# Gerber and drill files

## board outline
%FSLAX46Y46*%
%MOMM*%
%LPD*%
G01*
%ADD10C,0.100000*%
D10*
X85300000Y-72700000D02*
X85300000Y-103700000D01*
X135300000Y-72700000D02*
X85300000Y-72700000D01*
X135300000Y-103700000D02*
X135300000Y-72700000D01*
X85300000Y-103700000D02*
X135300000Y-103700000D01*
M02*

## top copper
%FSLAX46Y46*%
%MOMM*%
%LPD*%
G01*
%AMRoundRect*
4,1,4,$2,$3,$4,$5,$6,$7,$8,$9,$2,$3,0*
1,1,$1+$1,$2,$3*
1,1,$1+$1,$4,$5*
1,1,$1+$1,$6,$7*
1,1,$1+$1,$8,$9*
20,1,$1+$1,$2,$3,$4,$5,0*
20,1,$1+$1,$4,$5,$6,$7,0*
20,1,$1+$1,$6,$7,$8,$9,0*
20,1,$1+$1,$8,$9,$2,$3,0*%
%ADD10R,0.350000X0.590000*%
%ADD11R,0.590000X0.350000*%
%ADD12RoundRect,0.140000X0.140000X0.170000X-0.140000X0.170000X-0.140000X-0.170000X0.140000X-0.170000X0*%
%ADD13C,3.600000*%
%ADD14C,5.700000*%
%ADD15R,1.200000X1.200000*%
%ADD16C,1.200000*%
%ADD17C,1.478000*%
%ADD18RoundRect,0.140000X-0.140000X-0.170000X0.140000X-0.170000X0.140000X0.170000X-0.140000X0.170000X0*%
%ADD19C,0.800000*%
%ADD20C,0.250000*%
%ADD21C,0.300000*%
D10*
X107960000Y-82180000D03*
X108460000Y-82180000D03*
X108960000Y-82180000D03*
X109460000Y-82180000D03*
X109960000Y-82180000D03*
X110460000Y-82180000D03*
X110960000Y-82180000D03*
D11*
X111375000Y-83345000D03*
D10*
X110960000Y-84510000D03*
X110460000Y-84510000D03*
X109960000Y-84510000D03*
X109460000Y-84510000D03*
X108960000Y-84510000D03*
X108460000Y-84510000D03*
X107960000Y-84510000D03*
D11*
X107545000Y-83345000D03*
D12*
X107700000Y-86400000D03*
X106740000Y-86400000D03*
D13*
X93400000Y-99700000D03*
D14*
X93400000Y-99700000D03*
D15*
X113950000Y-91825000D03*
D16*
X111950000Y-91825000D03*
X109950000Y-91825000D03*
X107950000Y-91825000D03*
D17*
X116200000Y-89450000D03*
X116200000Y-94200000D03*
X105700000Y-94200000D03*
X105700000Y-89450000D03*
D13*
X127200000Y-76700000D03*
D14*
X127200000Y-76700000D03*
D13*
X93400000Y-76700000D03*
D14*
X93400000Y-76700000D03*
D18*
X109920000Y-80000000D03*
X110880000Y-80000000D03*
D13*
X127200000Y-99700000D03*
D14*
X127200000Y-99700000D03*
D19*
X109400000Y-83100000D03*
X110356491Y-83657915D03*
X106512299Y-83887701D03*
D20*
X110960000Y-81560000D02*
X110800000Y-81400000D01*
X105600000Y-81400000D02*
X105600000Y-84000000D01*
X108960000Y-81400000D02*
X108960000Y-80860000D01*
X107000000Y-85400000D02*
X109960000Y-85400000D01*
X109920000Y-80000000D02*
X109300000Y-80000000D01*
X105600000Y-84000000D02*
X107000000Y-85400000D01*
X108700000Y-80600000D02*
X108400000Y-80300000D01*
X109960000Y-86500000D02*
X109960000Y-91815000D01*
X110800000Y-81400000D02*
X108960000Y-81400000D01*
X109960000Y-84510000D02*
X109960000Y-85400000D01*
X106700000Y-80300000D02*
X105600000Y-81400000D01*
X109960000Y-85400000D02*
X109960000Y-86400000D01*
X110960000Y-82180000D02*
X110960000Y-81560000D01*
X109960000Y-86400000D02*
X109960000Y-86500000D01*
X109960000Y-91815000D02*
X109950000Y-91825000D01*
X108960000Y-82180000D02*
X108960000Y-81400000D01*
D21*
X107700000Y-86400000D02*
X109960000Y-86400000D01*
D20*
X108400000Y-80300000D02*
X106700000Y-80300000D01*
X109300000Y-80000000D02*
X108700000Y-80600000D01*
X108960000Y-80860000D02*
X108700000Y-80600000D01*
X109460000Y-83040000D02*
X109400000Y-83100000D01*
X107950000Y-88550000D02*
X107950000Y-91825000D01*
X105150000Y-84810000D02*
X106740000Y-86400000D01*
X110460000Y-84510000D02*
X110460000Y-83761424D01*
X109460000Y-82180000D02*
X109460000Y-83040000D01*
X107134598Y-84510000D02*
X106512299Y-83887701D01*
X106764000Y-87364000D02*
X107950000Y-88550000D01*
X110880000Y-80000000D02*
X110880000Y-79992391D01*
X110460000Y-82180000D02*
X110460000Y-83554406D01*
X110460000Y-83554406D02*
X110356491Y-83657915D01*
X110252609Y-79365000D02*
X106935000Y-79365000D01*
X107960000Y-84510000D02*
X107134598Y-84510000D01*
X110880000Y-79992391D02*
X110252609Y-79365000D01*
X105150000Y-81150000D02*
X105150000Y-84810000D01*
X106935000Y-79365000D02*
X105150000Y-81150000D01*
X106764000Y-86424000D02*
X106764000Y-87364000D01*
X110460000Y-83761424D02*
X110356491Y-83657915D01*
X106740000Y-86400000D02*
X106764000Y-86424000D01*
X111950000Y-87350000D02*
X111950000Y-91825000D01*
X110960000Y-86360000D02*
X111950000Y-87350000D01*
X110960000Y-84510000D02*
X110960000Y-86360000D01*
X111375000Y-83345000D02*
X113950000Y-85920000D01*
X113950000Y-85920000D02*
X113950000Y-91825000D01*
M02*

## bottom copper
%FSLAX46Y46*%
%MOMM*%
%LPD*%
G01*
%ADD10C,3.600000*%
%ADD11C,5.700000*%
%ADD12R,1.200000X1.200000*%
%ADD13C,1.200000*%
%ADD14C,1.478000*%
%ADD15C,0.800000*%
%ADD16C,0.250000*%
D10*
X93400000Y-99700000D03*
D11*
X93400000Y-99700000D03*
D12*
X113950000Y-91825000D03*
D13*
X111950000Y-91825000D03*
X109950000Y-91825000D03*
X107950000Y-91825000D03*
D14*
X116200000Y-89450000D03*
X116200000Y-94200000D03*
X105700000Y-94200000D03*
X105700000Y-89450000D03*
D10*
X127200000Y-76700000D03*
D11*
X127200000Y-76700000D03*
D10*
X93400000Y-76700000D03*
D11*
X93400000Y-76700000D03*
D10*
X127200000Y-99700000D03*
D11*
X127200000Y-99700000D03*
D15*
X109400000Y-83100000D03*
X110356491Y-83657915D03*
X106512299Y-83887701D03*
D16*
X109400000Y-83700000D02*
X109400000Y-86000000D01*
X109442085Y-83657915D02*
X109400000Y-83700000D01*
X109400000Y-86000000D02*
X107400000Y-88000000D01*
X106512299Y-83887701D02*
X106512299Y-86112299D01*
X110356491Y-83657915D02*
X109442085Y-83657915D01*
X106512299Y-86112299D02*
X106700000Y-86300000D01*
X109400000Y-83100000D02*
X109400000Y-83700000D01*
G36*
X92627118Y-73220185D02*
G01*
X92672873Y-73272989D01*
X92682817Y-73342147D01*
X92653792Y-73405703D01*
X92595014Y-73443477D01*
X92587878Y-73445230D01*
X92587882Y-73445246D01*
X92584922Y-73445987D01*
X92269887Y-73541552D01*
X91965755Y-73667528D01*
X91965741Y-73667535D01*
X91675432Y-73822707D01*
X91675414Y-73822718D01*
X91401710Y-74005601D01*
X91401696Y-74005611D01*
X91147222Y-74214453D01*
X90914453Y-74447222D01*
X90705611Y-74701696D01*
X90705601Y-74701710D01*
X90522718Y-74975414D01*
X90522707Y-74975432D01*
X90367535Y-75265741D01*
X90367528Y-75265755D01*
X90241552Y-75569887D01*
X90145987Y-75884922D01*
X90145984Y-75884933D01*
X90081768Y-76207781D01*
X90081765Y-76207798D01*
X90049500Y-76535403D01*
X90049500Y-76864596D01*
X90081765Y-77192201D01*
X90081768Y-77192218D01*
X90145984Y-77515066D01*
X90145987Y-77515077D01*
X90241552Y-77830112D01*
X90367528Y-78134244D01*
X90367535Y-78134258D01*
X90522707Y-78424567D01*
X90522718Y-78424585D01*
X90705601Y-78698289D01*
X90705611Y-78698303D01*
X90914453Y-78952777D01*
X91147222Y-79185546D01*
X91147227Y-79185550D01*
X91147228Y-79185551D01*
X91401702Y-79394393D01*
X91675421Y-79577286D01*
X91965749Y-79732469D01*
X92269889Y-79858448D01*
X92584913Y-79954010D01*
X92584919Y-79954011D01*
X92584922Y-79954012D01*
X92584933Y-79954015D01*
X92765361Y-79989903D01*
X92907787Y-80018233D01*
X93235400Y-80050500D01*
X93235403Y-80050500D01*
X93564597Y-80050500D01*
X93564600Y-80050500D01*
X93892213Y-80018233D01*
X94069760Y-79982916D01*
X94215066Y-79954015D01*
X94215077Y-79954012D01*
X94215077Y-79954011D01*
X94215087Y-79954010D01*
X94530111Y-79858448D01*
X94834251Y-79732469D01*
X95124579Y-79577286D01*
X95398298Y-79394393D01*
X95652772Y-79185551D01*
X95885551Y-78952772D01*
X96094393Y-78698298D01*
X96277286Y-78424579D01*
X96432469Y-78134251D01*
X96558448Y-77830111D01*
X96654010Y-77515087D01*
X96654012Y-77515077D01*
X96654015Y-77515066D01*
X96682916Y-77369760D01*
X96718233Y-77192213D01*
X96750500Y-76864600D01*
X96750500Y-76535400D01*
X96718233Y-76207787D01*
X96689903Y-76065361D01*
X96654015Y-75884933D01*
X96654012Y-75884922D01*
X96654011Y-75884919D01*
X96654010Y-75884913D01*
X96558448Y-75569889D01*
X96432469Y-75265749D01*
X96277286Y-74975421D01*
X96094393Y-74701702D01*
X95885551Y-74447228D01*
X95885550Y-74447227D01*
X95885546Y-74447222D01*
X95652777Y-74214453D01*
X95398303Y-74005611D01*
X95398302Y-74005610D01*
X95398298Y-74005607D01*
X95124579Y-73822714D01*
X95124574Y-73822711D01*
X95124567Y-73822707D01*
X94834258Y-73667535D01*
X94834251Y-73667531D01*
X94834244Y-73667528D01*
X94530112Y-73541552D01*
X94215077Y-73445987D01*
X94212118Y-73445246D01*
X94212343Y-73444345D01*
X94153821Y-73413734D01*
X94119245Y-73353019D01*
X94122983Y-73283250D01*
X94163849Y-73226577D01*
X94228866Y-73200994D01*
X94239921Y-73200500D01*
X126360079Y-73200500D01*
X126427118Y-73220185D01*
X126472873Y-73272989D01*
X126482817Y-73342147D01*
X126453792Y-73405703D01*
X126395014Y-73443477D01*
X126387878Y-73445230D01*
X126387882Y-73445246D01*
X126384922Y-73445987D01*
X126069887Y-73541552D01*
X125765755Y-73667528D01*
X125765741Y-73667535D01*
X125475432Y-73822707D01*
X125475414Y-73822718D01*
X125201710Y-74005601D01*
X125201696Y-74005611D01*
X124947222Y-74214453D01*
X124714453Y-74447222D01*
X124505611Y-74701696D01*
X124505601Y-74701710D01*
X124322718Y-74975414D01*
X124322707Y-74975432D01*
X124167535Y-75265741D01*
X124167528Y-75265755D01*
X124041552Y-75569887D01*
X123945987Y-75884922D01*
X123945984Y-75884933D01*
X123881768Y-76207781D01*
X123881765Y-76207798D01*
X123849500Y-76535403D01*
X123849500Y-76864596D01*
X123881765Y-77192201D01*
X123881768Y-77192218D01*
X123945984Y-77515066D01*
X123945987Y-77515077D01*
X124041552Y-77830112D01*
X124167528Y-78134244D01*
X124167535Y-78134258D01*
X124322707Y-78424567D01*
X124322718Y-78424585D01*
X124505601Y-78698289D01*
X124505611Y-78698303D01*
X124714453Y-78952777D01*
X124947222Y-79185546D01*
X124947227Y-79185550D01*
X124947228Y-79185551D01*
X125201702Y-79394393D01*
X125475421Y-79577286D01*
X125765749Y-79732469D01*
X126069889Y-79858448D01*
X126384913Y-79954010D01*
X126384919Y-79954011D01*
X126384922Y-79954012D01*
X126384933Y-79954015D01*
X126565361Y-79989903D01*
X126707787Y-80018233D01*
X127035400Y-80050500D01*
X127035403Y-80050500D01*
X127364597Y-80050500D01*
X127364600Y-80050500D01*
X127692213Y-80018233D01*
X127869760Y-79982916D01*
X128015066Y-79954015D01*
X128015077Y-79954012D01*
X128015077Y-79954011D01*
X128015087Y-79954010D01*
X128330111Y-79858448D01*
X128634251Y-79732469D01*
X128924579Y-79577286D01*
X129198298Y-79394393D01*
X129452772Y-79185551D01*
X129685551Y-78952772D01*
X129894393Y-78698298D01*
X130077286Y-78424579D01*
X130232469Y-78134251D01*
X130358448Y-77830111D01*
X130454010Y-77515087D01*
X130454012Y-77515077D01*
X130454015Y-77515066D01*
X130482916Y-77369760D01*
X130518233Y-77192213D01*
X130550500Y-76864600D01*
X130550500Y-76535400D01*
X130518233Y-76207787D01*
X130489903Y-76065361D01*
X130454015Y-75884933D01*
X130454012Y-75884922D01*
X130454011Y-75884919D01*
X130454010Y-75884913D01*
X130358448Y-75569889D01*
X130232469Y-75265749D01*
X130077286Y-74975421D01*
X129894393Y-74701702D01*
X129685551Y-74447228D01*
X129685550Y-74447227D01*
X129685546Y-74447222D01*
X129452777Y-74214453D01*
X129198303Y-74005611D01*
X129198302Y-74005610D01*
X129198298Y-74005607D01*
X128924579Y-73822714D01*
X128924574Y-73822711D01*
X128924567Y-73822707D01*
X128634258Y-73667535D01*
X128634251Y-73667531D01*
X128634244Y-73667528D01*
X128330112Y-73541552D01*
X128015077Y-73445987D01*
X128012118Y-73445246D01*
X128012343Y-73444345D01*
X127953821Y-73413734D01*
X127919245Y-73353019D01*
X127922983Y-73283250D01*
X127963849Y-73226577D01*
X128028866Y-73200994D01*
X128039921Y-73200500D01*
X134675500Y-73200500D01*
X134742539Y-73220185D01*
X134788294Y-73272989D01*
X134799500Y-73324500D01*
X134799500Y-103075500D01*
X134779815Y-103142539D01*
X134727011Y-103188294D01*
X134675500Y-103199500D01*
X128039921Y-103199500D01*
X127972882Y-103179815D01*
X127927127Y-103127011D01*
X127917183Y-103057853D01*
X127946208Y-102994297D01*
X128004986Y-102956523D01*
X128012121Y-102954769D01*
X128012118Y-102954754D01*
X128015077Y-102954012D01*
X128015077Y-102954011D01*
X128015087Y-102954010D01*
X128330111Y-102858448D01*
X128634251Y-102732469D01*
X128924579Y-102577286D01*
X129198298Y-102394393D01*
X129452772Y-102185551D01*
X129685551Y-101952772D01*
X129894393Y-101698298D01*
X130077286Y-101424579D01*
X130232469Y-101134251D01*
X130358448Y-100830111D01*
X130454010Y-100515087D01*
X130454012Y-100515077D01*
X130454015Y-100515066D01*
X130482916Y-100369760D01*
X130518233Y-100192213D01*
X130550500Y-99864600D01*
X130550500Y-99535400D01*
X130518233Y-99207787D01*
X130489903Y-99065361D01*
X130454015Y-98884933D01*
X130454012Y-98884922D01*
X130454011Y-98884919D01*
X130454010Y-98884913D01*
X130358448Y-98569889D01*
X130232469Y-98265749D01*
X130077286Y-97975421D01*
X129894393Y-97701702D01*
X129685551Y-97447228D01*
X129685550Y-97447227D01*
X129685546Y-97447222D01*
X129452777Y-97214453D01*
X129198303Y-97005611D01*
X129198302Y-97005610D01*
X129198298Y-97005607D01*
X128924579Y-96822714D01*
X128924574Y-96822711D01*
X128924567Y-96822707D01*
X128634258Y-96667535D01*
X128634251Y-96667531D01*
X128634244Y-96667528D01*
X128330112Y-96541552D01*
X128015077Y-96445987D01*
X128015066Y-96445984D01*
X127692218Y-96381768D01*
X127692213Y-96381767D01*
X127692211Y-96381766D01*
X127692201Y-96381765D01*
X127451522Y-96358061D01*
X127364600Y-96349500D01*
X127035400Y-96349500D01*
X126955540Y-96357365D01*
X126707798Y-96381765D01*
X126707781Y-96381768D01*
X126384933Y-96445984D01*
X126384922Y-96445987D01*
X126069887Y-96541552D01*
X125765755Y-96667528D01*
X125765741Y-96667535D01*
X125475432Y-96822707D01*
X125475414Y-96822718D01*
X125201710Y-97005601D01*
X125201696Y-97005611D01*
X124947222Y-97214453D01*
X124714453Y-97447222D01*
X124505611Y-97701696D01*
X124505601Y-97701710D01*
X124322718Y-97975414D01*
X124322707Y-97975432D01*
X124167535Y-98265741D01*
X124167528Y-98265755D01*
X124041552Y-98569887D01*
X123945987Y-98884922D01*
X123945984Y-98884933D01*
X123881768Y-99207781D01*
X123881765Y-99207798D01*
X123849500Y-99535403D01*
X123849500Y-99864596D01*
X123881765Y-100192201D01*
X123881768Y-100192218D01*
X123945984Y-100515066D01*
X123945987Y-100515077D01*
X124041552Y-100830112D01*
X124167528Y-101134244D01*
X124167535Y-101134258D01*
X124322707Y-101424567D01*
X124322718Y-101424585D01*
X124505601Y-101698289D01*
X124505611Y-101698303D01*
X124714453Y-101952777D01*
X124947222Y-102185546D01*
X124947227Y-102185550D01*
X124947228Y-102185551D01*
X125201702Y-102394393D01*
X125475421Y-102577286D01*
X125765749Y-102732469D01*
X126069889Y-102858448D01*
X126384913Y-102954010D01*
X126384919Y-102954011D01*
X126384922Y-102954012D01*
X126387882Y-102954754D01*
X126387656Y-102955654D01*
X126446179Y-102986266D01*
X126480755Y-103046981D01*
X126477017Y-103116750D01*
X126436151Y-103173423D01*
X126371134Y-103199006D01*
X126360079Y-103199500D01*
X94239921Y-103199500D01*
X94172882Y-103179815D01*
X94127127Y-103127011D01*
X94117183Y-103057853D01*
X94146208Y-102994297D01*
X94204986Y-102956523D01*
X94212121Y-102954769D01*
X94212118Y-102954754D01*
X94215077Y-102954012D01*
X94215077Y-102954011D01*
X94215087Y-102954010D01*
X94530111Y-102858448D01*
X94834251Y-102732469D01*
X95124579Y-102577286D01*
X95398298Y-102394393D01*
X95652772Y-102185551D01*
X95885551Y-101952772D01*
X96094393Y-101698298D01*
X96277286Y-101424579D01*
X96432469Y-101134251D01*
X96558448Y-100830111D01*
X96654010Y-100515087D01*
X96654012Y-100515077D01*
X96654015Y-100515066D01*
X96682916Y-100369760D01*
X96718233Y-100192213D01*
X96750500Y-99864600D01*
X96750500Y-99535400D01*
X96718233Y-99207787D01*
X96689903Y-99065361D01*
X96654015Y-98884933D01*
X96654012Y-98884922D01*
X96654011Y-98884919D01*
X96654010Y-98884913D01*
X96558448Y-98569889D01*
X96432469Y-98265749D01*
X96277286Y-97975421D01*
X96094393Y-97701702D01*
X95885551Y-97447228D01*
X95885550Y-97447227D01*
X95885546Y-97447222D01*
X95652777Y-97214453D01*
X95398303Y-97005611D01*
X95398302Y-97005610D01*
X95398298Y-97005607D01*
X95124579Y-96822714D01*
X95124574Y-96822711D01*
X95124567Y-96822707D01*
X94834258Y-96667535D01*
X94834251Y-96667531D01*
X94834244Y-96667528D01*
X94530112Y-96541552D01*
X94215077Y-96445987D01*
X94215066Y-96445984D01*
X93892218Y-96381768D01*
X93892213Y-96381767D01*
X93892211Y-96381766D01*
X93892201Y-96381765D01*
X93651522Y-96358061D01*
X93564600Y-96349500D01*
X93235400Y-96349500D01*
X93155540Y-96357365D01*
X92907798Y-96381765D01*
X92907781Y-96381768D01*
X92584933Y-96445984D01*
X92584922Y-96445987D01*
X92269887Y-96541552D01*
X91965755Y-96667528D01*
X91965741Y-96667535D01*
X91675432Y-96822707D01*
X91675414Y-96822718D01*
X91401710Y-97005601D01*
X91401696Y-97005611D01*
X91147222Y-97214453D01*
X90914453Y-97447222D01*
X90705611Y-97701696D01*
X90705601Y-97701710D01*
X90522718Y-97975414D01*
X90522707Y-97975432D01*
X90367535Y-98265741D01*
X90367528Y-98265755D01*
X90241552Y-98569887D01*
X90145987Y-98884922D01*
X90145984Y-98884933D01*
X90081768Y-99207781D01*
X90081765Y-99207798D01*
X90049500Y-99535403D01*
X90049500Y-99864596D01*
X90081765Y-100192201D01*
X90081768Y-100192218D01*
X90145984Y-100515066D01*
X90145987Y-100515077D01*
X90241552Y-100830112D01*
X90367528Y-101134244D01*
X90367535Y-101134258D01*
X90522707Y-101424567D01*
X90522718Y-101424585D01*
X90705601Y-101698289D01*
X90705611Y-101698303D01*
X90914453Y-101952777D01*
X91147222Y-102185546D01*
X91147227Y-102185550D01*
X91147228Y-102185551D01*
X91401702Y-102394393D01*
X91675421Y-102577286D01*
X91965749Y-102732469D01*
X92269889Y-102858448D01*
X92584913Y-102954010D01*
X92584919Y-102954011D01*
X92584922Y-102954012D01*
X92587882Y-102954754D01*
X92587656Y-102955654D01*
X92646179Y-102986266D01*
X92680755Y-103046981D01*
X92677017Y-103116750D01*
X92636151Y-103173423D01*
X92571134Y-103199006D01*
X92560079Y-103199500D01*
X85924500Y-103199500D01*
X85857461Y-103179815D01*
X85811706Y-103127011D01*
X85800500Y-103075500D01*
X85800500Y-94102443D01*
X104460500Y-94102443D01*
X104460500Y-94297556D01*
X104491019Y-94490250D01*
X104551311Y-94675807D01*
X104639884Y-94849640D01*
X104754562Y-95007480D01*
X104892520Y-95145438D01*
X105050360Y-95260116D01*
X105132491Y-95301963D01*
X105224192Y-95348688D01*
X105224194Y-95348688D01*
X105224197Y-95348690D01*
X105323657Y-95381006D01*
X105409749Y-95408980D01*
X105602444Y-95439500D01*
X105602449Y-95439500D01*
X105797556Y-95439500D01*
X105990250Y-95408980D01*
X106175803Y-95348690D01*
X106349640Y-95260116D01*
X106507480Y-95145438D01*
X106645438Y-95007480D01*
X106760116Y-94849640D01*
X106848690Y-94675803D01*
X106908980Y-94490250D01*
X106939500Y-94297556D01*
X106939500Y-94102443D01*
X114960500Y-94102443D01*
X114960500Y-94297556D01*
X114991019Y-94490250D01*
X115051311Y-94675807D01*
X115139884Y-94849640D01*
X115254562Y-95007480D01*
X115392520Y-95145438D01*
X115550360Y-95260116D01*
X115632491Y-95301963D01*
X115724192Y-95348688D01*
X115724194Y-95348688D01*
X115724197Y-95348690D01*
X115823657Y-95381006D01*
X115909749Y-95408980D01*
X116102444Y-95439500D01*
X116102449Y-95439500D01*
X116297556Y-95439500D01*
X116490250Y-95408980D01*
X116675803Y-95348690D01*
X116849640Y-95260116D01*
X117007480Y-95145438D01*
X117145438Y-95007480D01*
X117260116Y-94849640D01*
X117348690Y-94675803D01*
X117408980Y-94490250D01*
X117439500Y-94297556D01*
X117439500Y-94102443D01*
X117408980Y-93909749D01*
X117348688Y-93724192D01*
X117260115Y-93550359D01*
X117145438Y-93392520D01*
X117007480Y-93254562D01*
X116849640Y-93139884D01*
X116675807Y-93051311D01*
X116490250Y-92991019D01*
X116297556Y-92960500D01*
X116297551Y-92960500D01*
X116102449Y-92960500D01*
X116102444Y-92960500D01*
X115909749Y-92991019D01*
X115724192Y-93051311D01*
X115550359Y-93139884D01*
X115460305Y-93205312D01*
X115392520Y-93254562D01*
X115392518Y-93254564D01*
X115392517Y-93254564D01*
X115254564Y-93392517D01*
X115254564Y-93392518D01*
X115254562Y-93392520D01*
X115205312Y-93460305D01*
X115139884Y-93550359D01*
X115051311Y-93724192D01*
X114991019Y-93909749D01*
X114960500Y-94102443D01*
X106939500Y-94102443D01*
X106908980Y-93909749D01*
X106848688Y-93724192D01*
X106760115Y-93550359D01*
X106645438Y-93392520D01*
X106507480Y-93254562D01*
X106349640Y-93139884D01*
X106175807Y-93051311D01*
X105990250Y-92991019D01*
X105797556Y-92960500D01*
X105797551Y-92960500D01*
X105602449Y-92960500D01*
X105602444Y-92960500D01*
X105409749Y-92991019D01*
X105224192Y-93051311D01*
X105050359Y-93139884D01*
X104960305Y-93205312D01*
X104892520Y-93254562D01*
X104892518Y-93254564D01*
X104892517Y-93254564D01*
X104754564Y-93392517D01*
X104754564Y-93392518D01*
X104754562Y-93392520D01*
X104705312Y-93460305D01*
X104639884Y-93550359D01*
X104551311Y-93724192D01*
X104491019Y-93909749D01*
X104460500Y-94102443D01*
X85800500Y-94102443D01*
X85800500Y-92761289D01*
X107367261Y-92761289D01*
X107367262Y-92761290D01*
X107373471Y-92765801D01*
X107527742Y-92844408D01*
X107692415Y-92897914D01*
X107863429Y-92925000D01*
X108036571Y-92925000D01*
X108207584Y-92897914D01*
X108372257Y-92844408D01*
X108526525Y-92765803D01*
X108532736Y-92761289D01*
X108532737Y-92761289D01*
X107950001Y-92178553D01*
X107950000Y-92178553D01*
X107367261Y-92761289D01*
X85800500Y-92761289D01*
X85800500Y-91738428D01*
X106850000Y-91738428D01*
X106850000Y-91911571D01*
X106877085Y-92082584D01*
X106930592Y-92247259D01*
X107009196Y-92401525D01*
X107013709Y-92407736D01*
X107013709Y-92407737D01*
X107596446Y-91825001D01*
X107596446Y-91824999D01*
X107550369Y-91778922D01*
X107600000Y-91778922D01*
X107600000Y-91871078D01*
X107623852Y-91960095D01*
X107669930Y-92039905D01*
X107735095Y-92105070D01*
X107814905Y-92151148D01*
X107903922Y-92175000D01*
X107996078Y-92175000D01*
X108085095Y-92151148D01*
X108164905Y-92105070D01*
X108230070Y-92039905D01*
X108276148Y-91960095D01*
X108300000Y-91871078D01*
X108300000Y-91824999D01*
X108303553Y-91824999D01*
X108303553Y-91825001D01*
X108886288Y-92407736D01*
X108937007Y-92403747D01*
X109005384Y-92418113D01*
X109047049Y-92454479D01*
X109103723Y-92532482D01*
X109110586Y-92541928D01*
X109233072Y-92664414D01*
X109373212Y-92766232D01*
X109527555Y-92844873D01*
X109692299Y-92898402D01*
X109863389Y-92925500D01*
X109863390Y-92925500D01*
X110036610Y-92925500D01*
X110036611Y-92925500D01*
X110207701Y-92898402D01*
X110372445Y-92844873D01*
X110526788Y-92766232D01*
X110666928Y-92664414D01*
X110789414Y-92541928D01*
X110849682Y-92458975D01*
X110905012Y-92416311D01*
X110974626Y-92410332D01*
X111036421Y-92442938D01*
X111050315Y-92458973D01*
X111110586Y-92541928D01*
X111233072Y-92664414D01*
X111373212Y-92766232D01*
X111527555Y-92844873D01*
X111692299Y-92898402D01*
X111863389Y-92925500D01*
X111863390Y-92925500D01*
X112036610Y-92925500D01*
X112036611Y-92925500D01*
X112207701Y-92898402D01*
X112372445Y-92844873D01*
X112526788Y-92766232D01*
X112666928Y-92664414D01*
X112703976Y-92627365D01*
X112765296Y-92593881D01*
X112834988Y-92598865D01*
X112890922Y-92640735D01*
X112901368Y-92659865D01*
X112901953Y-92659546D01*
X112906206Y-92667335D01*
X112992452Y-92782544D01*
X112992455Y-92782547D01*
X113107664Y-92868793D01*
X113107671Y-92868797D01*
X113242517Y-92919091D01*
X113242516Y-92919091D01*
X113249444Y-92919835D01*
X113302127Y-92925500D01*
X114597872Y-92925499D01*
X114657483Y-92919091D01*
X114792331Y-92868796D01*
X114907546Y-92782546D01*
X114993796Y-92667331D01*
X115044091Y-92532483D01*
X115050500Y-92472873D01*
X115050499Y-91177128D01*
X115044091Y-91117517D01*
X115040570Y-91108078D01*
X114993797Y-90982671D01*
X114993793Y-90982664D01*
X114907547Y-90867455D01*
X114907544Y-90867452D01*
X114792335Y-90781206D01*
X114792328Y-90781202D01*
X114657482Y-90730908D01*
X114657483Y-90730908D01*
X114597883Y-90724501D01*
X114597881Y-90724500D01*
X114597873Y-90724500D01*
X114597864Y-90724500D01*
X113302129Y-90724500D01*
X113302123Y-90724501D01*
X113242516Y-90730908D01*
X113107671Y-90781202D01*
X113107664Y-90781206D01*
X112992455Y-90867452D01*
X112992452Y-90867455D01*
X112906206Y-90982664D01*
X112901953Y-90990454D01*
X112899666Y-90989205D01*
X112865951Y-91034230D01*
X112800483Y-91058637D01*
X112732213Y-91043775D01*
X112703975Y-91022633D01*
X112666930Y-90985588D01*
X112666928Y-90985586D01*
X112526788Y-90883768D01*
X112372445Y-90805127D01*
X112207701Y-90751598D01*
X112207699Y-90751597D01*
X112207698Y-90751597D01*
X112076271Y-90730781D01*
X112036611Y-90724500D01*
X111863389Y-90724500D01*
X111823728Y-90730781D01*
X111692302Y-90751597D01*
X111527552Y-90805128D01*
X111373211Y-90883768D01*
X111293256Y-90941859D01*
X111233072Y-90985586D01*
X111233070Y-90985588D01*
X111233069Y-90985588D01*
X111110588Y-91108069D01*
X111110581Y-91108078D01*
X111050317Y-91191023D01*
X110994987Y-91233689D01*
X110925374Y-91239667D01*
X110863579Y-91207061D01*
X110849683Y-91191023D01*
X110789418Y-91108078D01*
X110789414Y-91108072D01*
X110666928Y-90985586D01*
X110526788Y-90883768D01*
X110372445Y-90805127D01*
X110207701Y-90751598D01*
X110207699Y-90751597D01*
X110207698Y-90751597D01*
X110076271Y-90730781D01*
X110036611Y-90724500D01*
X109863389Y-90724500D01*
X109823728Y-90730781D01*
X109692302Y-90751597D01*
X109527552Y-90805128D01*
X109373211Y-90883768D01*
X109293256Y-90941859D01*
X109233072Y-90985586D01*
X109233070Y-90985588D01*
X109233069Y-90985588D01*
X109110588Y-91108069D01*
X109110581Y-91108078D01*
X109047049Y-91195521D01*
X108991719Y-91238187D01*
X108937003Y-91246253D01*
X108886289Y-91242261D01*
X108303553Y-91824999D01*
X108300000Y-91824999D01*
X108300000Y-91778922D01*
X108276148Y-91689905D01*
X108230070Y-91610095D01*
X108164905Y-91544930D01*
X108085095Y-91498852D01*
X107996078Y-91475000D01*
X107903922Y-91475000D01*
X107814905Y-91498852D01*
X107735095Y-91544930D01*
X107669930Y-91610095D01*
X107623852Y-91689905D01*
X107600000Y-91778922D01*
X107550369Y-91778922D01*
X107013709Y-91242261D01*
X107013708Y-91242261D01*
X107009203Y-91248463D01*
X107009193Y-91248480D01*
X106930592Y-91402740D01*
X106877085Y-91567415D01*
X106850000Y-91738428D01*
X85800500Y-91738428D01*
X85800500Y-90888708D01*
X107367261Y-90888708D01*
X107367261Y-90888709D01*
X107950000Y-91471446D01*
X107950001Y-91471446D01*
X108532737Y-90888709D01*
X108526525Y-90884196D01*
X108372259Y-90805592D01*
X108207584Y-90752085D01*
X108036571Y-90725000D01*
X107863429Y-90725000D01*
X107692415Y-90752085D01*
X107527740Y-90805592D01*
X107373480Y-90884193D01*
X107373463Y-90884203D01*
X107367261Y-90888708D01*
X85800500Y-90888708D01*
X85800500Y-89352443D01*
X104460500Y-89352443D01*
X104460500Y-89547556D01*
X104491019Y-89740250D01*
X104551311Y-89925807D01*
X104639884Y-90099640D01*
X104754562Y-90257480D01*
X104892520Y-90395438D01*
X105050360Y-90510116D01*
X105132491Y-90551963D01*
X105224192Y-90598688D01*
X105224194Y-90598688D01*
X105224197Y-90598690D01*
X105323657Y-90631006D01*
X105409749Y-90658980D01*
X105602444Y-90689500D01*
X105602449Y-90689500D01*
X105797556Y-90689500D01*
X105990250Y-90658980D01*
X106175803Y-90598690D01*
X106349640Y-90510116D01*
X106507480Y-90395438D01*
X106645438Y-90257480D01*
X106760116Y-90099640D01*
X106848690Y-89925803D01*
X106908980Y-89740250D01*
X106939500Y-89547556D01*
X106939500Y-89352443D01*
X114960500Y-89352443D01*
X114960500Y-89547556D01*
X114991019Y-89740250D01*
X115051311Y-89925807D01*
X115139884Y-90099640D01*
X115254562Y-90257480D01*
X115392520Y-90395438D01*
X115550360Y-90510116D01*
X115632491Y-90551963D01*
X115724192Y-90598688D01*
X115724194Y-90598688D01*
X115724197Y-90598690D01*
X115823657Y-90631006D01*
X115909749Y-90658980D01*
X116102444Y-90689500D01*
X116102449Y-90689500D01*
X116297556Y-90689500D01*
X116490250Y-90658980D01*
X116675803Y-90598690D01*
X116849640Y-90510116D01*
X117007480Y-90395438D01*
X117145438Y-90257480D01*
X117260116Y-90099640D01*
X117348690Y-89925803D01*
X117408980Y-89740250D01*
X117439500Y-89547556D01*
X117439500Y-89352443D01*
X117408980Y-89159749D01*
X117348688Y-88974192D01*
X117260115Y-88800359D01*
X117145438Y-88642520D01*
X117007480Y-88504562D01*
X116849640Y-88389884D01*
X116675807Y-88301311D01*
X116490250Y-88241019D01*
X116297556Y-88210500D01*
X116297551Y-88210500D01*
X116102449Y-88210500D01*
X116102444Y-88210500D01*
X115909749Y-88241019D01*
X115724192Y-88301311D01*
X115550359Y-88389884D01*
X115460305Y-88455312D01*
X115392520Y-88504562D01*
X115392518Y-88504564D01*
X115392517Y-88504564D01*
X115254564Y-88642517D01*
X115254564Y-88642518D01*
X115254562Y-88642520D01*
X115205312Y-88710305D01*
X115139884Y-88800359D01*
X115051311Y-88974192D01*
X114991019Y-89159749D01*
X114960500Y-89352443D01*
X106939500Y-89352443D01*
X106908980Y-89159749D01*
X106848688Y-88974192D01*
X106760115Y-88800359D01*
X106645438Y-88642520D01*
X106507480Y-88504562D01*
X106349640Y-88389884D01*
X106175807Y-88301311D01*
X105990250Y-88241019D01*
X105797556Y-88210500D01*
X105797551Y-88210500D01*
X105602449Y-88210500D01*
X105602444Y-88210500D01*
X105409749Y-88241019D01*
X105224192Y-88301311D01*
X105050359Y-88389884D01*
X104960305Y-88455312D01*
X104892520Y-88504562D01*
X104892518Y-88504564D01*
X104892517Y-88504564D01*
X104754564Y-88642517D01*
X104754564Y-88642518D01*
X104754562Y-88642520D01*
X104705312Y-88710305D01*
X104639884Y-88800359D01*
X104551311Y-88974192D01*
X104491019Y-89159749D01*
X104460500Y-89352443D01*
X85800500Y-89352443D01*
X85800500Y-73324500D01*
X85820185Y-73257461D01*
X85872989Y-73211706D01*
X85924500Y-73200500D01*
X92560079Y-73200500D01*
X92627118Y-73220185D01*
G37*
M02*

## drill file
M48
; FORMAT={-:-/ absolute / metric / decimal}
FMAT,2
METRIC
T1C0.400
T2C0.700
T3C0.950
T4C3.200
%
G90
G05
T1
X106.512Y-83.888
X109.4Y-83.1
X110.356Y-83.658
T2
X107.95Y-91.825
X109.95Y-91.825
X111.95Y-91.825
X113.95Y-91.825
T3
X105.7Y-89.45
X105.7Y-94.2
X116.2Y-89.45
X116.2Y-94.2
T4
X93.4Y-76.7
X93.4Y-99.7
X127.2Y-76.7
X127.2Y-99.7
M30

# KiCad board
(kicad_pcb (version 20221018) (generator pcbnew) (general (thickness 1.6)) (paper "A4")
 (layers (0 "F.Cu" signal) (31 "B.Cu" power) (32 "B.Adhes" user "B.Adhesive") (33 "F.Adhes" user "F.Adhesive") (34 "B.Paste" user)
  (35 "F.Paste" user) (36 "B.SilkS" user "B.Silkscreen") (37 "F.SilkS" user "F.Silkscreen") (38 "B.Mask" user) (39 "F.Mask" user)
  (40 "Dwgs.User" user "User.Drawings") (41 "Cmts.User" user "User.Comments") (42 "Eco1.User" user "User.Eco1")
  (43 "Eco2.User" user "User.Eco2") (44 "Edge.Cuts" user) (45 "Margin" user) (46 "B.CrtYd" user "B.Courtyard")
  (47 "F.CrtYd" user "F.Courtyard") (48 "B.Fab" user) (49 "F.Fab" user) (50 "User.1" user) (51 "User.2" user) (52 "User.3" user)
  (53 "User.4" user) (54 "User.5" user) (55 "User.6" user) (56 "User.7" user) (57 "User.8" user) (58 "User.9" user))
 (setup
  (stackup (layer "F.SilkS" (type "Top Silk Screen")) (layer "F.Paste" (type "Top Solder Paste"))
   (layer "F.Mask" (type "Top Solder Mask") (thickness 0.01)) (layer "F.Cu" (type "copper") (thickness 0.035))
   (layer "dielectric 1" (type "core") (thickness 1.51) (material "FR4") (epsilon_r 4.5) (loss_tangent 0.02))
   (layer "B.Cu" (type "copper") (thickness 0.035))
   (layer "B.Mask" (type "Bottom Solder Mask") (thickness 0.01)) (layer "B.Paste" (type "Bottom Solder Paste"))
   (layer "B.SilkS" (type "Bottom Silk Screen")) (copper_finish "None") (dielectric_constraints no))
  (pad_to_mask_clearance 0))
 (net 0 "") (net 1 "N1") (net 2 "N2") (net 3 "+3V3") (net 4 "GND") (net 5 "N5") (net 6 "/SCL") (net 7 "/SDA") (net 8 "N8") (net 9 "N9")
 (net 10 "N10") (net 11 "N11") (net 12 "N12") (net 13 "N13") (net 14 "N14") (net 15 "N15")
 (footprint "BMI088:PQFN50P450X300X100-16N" (layer "F.Cu") (at 109.46 83.345)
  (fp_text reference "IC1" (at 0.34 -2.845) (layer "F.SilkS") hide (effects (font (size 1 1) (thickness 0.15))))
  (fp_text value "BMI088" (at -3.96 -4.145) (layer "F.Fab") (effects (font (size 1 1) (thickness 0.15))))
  (pad "1" smd rect (at -1.5 -1.165 270) (size 0.59 0.35) (layers "F.Cu" "F.Paste" "F.Mask") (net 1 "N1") (solder_mask_margin 0.102))
  (pad "2" smd rect (at -1 -1.165 270) (size 0.59 0.35) (layers "F.Cu" "F.Paste" "F.Mask") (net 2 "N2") (solder_mask_margin 0.102))
  (pad "3" smd rect (at -0.5 -1.165 270) (size 0.59 0.35) (layers "F.Cu" "F.Paste" "F.Mask") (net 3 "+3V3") (solder_mask_margin 0.102))
  (pad "4" smd rect (at 0 -1.165 270) (size 0.59 0.35) (layers "F.Cu" "F.Paste" "F.Mask") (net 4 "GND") (solder_mask_margin 0.102))
  (pad "5" smd rect (at 0.5 -1.165 270) (size 0.59 0.35) (layers "F.Cu" "F.Paste" "F.Mask") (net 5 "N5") (solder_mask_margin 0.102))
  (pad "6" smd rect (at 1 -1.165 270) (size 0.59 0.35) (layers "F.Cu" "F.Paste" "F.Mask") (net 4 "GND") (solder_mask_margin 0.102))
  (pad "7" smd rect (at 1.5 -1.165 270) (size 0.59 0.35) (layers "F.Cu" "F.Paste" "F.Mask") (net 3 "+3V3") (solder_mask_margin 0.102))
  (pad "8" smd rect (at 1.915 0 180) (size 0.59 0.35) (layers "F.Cu" "F.Paste" "F.Mask") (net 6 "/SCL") (solder_mask_margin 0.102))
  (pad "9" smd rect (at 1.5 1.165 90) (size 0.59 0.35) (layers "F.Cu" "F.Paste" "F.Mask") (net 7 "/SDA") (solder_mask_margin 0.102))
  (pad "10" smd rect (at 1 1.165 90) (size 0.59 0.35) (layers "F.Cu" "F.Paste" "F.Mask") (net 4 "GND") (solder_mask_margin 0.102))
  (pad "11" smd rect (at 0.5 1.165 90) (size 0.59 0.35) (layers "F.Cu" "F.Paste" "F.Mask") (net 3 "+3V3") (solder_mask_margin 0.102))
  (pad "12" smd rect (at 0 1.165 90) (size 0.59 0.35) (layers "F.Cu" "F.Paste" "F.Mask") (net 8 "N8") (solder_mask_margin 0.102))
  (pad "13" smd rect (at -0.5 1.165 90) (size 0.59 0.35) (layers "F.Cu" "F.Paste" "F.Mask") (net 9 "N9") (solder_mask_margin 0.102))
  (pad "14" smd rect (at -1 1.165 90) (size 0.59 0.35) (layers "F.Cu" "F.Paste" "F.Mask") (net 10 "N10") (solder_mask_margin 0.102))
  (pad "15" smd rect (at -1.5 1.165 90) (size 0.59 0.35) (layers "F.Cu" "F.Paste" "F.Mask") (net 4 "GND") (solder_mask_margin 0.102))
  (pad "16" smd rect (at -1.915 0) (size 0.59 0.35) (layers "F.Cu" "F.Paste" "F.Mask") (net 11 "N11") (solder_mask_margin 0.102)))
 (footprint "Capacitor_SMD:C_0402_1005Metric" (layer "F.Cu") (at 107.22 86.4 180)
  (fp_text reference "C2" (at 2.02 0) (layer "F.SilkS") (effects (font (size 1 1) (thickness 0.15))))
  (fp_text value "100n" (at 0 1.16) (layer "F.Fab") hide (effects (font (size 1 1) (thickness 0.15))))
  (pad "1" smd roundrect (at -0.48 0 180) (size 0.56 0.62) (layers "F.Cu" "F.Paste" "F.Mask") (roundrect_rratio 0.25) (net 3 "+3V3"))
  (pad "2" smd roundrect (at 0.48 0 180) (size 0.56 0.62) (layers "F.Cu" "F.Paste" "F.Mask") (roundrect_rratio 0.25) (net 4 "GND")))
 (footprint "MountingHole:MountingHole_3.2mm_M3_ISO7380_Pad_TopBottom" (layer "F.Cu") (at 93.4 99.7)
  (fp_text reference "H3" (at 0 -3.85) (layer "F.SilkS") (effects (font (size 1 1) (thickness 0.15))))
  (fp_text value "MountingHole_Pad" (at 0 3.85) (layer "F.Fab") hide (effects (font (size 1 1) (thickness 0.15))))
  (pad "1" thru_hole circle (at 0 0) (size 3.6 3.6) (drill 3.2) (layers "*.Cu" "*.Mask"))
  (pad "1" connect circle (at 0 0) (size 5.7 5.7) (layers "F.Cu" "F.Mask"))
  (pad "1" connect circle (at 0 0) (size 5.7 5.7) (layers "B.Cu" "B.Mask")))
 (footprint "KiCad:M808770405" (layer "F.Cu") (at 113.95 91.825)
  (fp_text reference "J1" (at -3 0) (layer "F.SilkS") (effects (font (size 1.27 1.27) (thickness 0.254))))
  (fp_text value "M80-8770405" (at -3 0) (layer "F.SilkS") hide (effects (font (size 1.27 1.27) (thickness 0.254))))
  (pad "1" thru_hole rect (at 0 0) (size 1.2 1.2) (drill 0.7) (layers "*.Cu" "*.Mask") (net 6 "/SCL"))
  (pad "2" thru_hole circle (at -2 0) (size 1.2 1.2) (drill 0.7) (layers "*.Cu" "*.Mask") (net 7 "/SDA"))
  (pad "3" thru_hole circle (at -4 0) (size 1.2 1.2) (drill 0.7) (layers "*.Cu" "*.Mask") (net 3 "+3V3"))
  (pad "4" thru_hole circle (at -6 0) (size 1.2 1.2) (drill 0.7) (layers "*.Cu" "*.Mask") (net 4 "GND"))
  (pad "MH1" thru_hole circle (at 2.25 -2.375) (size 1.478 1.478) (drill 0.95) (layers "*.Cu" "*.Mask") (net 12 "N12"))
  (pad "MH2" thru_hole circle (at 2.25 2.375) (size 1.478 1.478) (drill 0.95) (layers "*.Cu" "*.Mask") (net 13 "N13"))
  (pad "MH3" thru_hole circle (at -8.25 2.375) (size 1.478 1.478) (drill 0.95) (layers "*.Cu" "*.Mask") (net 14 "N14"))
  (pad "MH4" thru_hole circle (at -8.25 -2.375) (size 1.478 1.478) (drill 0.95) (layers "*.Cu" "*.Mask") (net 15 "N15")))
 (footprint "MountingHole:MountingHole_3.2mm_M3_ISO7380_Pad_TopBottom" (layer "F.Cu") (at 127.2 76.7)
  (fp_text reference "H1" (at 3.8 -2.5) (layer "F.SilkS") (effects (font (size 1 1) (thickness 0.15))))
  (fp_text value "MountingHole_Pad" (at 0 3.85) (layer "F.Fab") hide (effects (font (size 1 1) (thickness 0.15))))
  (pad "1" thru_hole circle (at 0 0) (size 3.6 3.6) (drill 3.2) (layers "*.Cu" "*.Mask"))
  (pad "1" connect circle (at 0 0) (size 5.7 5.7) (layers "F.Cu" "F.Mask"))
  (pad "1" connect circle (at 0 0) (size 5.7 5.7) (layers "B.Cu" "B.Mask")))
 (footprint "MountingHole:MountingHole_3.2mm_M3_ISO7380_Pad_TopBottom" (layer "F.Cu") (at 93.4 76.7)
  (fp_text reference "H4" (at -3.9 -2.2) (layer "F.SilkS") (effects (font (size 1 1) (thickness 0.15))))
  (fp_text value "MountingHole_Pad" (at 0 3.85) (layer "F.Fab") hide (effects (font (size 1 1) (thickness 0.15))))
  (pad "1" thru_hole circle (at 0 0) (size 3.6 3.6) (drill 3.2) (layers "*.Cu" "*.Mask"))
  (pad "1" connect circle (at 0 0) (size 5.7 5.7) (layers "F.Cu" "F.Mask"))
  (pad "1" connect circle (at 0 0) (size 5.7 5.7) (layers "B.Cu" "B.Mask")))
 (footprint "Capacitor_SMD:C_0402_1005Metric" (layer "F.Cu") (at 110.4 80)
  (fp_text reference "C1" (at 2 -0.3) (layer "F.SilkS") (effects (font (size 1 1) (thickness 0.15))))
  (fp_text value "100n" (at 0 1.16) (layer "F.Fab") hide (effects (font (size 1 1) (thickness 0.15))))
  (pad "1" smd roundrect (at -0.48 0) (size 0.56 0.62) (layers "F.Cu" "F.Paste" "F.Mask") (roundrect_rratio 0.25) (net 3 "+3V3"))
  (pad "2" smd roundrect (at 0.48 0) (size 0.56 0.62) (layers "F.Cu" "F.Paste" "F.Mask") (roundrect_rratio 0.25) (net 4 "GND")))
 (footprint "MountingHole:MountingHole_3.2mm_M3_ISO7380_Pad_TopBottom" (layer "F.Cu") (at 127.2 99.7)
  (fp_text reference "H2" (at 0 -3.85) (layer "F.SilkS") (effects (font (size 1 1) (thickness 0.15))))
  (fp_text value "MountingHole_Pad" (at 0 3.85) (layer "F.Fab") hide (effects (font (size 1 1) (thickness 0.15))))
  (pad "1" thru_hole circle (at 0 0) (size 3.6 3.6) (drill 3.2) (layers "*.Cu" "*.Mask"))
  (pad "1" connect circle (at 0 0) (size 5.7 5.7) (layers "F.Cu" "F.Mask"))
  (pad "1" connect circle (at 0 0) (size 5.7 5.7) (layers "B.Cu" "B.Mask")))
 (gr_line (start 85.3 72.7) (end 85.3 103.7) (stroke (width 0.1) (type default)) (layer "Edge.Cuts"))
 (gr_line (start 135.3 72.7) (end 85.3 72.7) (stroke (width 0.1) (type default)) (layer "Edge.Cuts"))
 (gr_line (start 135.3 103.7) (end 135.3 72.7) (stroke (width 0.1) (type default)) (layer "Edge.Cuts"))
 (gr_line (start 85.3 103.7) (end 135.3 103.7) (stroke (width 0.1) (type default)) (layer "Edge.Cuts"))
 (segment (start 110.96 81.56) (end 110.8 81.4) (width 0.25) (layer "F.Cu") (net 3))
 (segment (start 105.6 81.4) (end 105.6 84) (width 0.25) (layer "F.Cu") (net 3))
 (segment (start 108.96 81.4) (end 108.96 80.86) (width 0.25) (layer "F.Cu") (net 3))
 (segment (start 107 85.4) (end 109.96 85.4) (width 0.25) (layer "F.Cu") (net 3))
 (segment (start 109.92 80) (end 109.3 80) (width 0.25) (layer "F.Cu") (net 3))
 (segment (start 105.6 84) (end 107 85.4) (width 0.25) (layer "F.Cu") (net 3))
 (segment (start 108.7 80.6) (end 108.4 80.3) (width 0.25) (layer "F.Cu") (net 3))
 (segment (start 109.96 86.5) (end 109.96 91.815) (width 0.25) (layer "F.Cu") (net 3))
 (segment (start 110.8 81.4) (end 108.96 81.4) (width 0.25) (layer "F.Cu") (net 3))
 (segment (start 109.96 84.51) (end 109.96 85.4) (width 0.25) (layer "F.Cu") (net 3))
 (segment (start 106.7 80.3) (end 105.6 81.4) (width 0.25) (layer "F.Cu") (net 3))
 (segment (start 109.96 85.4) (end 109.96 86.4) (width 0.25) (layer "F.Cu") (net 3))
 (segment (start 110.96 82.18) (end 110.96 81.56) (width 0.25) (layer "F.Cu") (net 3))
 (segment (start 109.96 86.4) (end 109.96 86.5) (width 0.25) (layer "F.Cu") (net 3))
 (segment (start 109.96 91.815) (end 109.95 91.825) (width 0.25) (layer "F.Cu") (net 3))
 (segment (start 108.96 82.18) (end 108.96 81.4) (width 0.25) (layer "F.Cu") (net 3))
 (segment (start 107.7 86.4) (end 109.96 86.4) (width 0.3) (layer "F.Cu") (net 3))
 (segment (start 108.4 80.3) (end 106.7 80.3) (width 0.25) (layer "F.Cu") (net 3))
 (segment (start 109.3 80) (end 108.7 80.6) (width 0.25) (layer "F.Cu") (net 3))
 (segment (start 108.96 80.86) (end 108.7 80.6) (width 0.25) (layer "F.Cu") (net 3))
 (segment (start 109.46 83.04) (end 109.4 83.1) (width 0.25) (layer "F.Cu") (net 4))
 (segment (start 107.95 88.55) (end 107.95 91.825) (width 0.25) (layer "F.Cu") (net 4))
 (segment (start 105.15 84.81) (end 106.74 86.4) (width 0.25) (layer "F.Cu") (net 4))
 (segment (start 110.46 84.51) (end 110.46 83.761424) (width 0.25) (layer "F.Cu") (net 4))
 (segment (start 109.46 82.18) (end 109.46 83.04) (width 0.25) (layer "F.Cu") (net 4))
 (segment (start 107.134598 84.51) (end 106.512299 83.887701) (width 0.25) (layer "F.Cu") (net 4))
 (segment (start 106.764 87.364) (end 107.95 88.55) (width 0.25) (layer "F.Cu") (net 4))
 (segment (start 110.88 80) (end 110.88 79.992391) (width 0.25) (layer "F.Cu") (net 4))
 (segment (start 110.46 82.18) (end 110.46 83.554406) (width 0.25) (layer "F.Cu") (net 4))
 (segment (start 110.46 83.554406) (end 110.356491 83.657915) (width 0.25) (layer "F.Cu") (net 4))
 (segment (start 110.252609 79.365) (end 106.935 79.365) (width 0.25) (layer "F.Cu") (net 4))
 (segment (start 107.96 84.51) (end 107.134598 84.51) (width 0.25) (layer "F.Cu") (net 4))
 (segment (start 110.88 79.992391) (end 110.252609 79.365) (width 0.25) (layer "F.Cu") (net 4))
 (segment (start 105.15 81.15) (end 105.15 84.81) (width 0.25) (layer "F.Cu") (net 4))
 (segment (start 106.935 79.365) (end 105.15 81.15) (width 0.25) (layer "F.Cu") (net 4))
 (segment (start 106.764 86.424) (end 106.764 87.364) (width 0.25) (layer "F.Cu") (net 4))
 (segment (start 110.46 83.761424) (end 110.356491 83.657915) (width 0.25) (layer "F.Cu") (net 4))
 (segment (start 106.74 86.4) (end 106.764 86.424) (width 0.25) (layer "F.Cu") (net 4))
 (via (at 109.4 83.1) (size 0.8) (drill 0.4) (layers "F.Cu" "B.Cu") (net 4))
 (via (at 110.356491 83.657915) (size 0.8) (drill 0.4) (layers "F.Cu" "B.Cu") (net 4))
 (via (at 106.512299 83.887701) (size 0.8) (drill 0.4) (layers "F.Cu" "B.Cu") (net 4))
 (segment (start 109.4 83.7) (end 109.4 86) (width 0.25) (layer "B.Cu") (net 4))
 (segment (start 109.442085 83.657915) (end 109.4 83.7) (width 0.25) (layer "B.Cu") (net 4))
 (segment (start 109.4 86) (end 107.4 88) (width 0.25) (layer "B.Cu") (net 4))
 (segment (start 106.512299 83.887701) (end 106.512299 86.112299) (width 0.25) (layer "B.Cu") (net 4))
 (segment (start 110.356491 83.657915) (end 109.442085 83.657915) (width 0.25) (layer "B.Cu") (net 4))
 (segment (start 106.512299 86.112299) (end 106.7 86.3) (width 0.25) (layer "B.Cu") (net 4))
 (segment (start 109.4 83.1) (end 109.4 83.7) (width 0.25) (layer "B.Cu") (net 4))
 (segment (start 111.95 87.35) (end 111.95 91.825) (width 0.25) (layer "F.Cu") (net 7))
 (segment (start 110.96 86.36) (end 111.95 87.35) (width 0.25) (layer "F.Cu") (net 7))
 (segment (start 110.96 84.51) (end 110.96 86.36) (width 0.25) (layer "F.Cu") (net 7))
 (segment (start 111.375 83.345) (end 113.95 85.92) (width 0.25) (layer "F.Cu") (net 6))
 (segment (start 113.95 85.92) (end 113.95 91.825) (width 0.25) (layer "F.Cu") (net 6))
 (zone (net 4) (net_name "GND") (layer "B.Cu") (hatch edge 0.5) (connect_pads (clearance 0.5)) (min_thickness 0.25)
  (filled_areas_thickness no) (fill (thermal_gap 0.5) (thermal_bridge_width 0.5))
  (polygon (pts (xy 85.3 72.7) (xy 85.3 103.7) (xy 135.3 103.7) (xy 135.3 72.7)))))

